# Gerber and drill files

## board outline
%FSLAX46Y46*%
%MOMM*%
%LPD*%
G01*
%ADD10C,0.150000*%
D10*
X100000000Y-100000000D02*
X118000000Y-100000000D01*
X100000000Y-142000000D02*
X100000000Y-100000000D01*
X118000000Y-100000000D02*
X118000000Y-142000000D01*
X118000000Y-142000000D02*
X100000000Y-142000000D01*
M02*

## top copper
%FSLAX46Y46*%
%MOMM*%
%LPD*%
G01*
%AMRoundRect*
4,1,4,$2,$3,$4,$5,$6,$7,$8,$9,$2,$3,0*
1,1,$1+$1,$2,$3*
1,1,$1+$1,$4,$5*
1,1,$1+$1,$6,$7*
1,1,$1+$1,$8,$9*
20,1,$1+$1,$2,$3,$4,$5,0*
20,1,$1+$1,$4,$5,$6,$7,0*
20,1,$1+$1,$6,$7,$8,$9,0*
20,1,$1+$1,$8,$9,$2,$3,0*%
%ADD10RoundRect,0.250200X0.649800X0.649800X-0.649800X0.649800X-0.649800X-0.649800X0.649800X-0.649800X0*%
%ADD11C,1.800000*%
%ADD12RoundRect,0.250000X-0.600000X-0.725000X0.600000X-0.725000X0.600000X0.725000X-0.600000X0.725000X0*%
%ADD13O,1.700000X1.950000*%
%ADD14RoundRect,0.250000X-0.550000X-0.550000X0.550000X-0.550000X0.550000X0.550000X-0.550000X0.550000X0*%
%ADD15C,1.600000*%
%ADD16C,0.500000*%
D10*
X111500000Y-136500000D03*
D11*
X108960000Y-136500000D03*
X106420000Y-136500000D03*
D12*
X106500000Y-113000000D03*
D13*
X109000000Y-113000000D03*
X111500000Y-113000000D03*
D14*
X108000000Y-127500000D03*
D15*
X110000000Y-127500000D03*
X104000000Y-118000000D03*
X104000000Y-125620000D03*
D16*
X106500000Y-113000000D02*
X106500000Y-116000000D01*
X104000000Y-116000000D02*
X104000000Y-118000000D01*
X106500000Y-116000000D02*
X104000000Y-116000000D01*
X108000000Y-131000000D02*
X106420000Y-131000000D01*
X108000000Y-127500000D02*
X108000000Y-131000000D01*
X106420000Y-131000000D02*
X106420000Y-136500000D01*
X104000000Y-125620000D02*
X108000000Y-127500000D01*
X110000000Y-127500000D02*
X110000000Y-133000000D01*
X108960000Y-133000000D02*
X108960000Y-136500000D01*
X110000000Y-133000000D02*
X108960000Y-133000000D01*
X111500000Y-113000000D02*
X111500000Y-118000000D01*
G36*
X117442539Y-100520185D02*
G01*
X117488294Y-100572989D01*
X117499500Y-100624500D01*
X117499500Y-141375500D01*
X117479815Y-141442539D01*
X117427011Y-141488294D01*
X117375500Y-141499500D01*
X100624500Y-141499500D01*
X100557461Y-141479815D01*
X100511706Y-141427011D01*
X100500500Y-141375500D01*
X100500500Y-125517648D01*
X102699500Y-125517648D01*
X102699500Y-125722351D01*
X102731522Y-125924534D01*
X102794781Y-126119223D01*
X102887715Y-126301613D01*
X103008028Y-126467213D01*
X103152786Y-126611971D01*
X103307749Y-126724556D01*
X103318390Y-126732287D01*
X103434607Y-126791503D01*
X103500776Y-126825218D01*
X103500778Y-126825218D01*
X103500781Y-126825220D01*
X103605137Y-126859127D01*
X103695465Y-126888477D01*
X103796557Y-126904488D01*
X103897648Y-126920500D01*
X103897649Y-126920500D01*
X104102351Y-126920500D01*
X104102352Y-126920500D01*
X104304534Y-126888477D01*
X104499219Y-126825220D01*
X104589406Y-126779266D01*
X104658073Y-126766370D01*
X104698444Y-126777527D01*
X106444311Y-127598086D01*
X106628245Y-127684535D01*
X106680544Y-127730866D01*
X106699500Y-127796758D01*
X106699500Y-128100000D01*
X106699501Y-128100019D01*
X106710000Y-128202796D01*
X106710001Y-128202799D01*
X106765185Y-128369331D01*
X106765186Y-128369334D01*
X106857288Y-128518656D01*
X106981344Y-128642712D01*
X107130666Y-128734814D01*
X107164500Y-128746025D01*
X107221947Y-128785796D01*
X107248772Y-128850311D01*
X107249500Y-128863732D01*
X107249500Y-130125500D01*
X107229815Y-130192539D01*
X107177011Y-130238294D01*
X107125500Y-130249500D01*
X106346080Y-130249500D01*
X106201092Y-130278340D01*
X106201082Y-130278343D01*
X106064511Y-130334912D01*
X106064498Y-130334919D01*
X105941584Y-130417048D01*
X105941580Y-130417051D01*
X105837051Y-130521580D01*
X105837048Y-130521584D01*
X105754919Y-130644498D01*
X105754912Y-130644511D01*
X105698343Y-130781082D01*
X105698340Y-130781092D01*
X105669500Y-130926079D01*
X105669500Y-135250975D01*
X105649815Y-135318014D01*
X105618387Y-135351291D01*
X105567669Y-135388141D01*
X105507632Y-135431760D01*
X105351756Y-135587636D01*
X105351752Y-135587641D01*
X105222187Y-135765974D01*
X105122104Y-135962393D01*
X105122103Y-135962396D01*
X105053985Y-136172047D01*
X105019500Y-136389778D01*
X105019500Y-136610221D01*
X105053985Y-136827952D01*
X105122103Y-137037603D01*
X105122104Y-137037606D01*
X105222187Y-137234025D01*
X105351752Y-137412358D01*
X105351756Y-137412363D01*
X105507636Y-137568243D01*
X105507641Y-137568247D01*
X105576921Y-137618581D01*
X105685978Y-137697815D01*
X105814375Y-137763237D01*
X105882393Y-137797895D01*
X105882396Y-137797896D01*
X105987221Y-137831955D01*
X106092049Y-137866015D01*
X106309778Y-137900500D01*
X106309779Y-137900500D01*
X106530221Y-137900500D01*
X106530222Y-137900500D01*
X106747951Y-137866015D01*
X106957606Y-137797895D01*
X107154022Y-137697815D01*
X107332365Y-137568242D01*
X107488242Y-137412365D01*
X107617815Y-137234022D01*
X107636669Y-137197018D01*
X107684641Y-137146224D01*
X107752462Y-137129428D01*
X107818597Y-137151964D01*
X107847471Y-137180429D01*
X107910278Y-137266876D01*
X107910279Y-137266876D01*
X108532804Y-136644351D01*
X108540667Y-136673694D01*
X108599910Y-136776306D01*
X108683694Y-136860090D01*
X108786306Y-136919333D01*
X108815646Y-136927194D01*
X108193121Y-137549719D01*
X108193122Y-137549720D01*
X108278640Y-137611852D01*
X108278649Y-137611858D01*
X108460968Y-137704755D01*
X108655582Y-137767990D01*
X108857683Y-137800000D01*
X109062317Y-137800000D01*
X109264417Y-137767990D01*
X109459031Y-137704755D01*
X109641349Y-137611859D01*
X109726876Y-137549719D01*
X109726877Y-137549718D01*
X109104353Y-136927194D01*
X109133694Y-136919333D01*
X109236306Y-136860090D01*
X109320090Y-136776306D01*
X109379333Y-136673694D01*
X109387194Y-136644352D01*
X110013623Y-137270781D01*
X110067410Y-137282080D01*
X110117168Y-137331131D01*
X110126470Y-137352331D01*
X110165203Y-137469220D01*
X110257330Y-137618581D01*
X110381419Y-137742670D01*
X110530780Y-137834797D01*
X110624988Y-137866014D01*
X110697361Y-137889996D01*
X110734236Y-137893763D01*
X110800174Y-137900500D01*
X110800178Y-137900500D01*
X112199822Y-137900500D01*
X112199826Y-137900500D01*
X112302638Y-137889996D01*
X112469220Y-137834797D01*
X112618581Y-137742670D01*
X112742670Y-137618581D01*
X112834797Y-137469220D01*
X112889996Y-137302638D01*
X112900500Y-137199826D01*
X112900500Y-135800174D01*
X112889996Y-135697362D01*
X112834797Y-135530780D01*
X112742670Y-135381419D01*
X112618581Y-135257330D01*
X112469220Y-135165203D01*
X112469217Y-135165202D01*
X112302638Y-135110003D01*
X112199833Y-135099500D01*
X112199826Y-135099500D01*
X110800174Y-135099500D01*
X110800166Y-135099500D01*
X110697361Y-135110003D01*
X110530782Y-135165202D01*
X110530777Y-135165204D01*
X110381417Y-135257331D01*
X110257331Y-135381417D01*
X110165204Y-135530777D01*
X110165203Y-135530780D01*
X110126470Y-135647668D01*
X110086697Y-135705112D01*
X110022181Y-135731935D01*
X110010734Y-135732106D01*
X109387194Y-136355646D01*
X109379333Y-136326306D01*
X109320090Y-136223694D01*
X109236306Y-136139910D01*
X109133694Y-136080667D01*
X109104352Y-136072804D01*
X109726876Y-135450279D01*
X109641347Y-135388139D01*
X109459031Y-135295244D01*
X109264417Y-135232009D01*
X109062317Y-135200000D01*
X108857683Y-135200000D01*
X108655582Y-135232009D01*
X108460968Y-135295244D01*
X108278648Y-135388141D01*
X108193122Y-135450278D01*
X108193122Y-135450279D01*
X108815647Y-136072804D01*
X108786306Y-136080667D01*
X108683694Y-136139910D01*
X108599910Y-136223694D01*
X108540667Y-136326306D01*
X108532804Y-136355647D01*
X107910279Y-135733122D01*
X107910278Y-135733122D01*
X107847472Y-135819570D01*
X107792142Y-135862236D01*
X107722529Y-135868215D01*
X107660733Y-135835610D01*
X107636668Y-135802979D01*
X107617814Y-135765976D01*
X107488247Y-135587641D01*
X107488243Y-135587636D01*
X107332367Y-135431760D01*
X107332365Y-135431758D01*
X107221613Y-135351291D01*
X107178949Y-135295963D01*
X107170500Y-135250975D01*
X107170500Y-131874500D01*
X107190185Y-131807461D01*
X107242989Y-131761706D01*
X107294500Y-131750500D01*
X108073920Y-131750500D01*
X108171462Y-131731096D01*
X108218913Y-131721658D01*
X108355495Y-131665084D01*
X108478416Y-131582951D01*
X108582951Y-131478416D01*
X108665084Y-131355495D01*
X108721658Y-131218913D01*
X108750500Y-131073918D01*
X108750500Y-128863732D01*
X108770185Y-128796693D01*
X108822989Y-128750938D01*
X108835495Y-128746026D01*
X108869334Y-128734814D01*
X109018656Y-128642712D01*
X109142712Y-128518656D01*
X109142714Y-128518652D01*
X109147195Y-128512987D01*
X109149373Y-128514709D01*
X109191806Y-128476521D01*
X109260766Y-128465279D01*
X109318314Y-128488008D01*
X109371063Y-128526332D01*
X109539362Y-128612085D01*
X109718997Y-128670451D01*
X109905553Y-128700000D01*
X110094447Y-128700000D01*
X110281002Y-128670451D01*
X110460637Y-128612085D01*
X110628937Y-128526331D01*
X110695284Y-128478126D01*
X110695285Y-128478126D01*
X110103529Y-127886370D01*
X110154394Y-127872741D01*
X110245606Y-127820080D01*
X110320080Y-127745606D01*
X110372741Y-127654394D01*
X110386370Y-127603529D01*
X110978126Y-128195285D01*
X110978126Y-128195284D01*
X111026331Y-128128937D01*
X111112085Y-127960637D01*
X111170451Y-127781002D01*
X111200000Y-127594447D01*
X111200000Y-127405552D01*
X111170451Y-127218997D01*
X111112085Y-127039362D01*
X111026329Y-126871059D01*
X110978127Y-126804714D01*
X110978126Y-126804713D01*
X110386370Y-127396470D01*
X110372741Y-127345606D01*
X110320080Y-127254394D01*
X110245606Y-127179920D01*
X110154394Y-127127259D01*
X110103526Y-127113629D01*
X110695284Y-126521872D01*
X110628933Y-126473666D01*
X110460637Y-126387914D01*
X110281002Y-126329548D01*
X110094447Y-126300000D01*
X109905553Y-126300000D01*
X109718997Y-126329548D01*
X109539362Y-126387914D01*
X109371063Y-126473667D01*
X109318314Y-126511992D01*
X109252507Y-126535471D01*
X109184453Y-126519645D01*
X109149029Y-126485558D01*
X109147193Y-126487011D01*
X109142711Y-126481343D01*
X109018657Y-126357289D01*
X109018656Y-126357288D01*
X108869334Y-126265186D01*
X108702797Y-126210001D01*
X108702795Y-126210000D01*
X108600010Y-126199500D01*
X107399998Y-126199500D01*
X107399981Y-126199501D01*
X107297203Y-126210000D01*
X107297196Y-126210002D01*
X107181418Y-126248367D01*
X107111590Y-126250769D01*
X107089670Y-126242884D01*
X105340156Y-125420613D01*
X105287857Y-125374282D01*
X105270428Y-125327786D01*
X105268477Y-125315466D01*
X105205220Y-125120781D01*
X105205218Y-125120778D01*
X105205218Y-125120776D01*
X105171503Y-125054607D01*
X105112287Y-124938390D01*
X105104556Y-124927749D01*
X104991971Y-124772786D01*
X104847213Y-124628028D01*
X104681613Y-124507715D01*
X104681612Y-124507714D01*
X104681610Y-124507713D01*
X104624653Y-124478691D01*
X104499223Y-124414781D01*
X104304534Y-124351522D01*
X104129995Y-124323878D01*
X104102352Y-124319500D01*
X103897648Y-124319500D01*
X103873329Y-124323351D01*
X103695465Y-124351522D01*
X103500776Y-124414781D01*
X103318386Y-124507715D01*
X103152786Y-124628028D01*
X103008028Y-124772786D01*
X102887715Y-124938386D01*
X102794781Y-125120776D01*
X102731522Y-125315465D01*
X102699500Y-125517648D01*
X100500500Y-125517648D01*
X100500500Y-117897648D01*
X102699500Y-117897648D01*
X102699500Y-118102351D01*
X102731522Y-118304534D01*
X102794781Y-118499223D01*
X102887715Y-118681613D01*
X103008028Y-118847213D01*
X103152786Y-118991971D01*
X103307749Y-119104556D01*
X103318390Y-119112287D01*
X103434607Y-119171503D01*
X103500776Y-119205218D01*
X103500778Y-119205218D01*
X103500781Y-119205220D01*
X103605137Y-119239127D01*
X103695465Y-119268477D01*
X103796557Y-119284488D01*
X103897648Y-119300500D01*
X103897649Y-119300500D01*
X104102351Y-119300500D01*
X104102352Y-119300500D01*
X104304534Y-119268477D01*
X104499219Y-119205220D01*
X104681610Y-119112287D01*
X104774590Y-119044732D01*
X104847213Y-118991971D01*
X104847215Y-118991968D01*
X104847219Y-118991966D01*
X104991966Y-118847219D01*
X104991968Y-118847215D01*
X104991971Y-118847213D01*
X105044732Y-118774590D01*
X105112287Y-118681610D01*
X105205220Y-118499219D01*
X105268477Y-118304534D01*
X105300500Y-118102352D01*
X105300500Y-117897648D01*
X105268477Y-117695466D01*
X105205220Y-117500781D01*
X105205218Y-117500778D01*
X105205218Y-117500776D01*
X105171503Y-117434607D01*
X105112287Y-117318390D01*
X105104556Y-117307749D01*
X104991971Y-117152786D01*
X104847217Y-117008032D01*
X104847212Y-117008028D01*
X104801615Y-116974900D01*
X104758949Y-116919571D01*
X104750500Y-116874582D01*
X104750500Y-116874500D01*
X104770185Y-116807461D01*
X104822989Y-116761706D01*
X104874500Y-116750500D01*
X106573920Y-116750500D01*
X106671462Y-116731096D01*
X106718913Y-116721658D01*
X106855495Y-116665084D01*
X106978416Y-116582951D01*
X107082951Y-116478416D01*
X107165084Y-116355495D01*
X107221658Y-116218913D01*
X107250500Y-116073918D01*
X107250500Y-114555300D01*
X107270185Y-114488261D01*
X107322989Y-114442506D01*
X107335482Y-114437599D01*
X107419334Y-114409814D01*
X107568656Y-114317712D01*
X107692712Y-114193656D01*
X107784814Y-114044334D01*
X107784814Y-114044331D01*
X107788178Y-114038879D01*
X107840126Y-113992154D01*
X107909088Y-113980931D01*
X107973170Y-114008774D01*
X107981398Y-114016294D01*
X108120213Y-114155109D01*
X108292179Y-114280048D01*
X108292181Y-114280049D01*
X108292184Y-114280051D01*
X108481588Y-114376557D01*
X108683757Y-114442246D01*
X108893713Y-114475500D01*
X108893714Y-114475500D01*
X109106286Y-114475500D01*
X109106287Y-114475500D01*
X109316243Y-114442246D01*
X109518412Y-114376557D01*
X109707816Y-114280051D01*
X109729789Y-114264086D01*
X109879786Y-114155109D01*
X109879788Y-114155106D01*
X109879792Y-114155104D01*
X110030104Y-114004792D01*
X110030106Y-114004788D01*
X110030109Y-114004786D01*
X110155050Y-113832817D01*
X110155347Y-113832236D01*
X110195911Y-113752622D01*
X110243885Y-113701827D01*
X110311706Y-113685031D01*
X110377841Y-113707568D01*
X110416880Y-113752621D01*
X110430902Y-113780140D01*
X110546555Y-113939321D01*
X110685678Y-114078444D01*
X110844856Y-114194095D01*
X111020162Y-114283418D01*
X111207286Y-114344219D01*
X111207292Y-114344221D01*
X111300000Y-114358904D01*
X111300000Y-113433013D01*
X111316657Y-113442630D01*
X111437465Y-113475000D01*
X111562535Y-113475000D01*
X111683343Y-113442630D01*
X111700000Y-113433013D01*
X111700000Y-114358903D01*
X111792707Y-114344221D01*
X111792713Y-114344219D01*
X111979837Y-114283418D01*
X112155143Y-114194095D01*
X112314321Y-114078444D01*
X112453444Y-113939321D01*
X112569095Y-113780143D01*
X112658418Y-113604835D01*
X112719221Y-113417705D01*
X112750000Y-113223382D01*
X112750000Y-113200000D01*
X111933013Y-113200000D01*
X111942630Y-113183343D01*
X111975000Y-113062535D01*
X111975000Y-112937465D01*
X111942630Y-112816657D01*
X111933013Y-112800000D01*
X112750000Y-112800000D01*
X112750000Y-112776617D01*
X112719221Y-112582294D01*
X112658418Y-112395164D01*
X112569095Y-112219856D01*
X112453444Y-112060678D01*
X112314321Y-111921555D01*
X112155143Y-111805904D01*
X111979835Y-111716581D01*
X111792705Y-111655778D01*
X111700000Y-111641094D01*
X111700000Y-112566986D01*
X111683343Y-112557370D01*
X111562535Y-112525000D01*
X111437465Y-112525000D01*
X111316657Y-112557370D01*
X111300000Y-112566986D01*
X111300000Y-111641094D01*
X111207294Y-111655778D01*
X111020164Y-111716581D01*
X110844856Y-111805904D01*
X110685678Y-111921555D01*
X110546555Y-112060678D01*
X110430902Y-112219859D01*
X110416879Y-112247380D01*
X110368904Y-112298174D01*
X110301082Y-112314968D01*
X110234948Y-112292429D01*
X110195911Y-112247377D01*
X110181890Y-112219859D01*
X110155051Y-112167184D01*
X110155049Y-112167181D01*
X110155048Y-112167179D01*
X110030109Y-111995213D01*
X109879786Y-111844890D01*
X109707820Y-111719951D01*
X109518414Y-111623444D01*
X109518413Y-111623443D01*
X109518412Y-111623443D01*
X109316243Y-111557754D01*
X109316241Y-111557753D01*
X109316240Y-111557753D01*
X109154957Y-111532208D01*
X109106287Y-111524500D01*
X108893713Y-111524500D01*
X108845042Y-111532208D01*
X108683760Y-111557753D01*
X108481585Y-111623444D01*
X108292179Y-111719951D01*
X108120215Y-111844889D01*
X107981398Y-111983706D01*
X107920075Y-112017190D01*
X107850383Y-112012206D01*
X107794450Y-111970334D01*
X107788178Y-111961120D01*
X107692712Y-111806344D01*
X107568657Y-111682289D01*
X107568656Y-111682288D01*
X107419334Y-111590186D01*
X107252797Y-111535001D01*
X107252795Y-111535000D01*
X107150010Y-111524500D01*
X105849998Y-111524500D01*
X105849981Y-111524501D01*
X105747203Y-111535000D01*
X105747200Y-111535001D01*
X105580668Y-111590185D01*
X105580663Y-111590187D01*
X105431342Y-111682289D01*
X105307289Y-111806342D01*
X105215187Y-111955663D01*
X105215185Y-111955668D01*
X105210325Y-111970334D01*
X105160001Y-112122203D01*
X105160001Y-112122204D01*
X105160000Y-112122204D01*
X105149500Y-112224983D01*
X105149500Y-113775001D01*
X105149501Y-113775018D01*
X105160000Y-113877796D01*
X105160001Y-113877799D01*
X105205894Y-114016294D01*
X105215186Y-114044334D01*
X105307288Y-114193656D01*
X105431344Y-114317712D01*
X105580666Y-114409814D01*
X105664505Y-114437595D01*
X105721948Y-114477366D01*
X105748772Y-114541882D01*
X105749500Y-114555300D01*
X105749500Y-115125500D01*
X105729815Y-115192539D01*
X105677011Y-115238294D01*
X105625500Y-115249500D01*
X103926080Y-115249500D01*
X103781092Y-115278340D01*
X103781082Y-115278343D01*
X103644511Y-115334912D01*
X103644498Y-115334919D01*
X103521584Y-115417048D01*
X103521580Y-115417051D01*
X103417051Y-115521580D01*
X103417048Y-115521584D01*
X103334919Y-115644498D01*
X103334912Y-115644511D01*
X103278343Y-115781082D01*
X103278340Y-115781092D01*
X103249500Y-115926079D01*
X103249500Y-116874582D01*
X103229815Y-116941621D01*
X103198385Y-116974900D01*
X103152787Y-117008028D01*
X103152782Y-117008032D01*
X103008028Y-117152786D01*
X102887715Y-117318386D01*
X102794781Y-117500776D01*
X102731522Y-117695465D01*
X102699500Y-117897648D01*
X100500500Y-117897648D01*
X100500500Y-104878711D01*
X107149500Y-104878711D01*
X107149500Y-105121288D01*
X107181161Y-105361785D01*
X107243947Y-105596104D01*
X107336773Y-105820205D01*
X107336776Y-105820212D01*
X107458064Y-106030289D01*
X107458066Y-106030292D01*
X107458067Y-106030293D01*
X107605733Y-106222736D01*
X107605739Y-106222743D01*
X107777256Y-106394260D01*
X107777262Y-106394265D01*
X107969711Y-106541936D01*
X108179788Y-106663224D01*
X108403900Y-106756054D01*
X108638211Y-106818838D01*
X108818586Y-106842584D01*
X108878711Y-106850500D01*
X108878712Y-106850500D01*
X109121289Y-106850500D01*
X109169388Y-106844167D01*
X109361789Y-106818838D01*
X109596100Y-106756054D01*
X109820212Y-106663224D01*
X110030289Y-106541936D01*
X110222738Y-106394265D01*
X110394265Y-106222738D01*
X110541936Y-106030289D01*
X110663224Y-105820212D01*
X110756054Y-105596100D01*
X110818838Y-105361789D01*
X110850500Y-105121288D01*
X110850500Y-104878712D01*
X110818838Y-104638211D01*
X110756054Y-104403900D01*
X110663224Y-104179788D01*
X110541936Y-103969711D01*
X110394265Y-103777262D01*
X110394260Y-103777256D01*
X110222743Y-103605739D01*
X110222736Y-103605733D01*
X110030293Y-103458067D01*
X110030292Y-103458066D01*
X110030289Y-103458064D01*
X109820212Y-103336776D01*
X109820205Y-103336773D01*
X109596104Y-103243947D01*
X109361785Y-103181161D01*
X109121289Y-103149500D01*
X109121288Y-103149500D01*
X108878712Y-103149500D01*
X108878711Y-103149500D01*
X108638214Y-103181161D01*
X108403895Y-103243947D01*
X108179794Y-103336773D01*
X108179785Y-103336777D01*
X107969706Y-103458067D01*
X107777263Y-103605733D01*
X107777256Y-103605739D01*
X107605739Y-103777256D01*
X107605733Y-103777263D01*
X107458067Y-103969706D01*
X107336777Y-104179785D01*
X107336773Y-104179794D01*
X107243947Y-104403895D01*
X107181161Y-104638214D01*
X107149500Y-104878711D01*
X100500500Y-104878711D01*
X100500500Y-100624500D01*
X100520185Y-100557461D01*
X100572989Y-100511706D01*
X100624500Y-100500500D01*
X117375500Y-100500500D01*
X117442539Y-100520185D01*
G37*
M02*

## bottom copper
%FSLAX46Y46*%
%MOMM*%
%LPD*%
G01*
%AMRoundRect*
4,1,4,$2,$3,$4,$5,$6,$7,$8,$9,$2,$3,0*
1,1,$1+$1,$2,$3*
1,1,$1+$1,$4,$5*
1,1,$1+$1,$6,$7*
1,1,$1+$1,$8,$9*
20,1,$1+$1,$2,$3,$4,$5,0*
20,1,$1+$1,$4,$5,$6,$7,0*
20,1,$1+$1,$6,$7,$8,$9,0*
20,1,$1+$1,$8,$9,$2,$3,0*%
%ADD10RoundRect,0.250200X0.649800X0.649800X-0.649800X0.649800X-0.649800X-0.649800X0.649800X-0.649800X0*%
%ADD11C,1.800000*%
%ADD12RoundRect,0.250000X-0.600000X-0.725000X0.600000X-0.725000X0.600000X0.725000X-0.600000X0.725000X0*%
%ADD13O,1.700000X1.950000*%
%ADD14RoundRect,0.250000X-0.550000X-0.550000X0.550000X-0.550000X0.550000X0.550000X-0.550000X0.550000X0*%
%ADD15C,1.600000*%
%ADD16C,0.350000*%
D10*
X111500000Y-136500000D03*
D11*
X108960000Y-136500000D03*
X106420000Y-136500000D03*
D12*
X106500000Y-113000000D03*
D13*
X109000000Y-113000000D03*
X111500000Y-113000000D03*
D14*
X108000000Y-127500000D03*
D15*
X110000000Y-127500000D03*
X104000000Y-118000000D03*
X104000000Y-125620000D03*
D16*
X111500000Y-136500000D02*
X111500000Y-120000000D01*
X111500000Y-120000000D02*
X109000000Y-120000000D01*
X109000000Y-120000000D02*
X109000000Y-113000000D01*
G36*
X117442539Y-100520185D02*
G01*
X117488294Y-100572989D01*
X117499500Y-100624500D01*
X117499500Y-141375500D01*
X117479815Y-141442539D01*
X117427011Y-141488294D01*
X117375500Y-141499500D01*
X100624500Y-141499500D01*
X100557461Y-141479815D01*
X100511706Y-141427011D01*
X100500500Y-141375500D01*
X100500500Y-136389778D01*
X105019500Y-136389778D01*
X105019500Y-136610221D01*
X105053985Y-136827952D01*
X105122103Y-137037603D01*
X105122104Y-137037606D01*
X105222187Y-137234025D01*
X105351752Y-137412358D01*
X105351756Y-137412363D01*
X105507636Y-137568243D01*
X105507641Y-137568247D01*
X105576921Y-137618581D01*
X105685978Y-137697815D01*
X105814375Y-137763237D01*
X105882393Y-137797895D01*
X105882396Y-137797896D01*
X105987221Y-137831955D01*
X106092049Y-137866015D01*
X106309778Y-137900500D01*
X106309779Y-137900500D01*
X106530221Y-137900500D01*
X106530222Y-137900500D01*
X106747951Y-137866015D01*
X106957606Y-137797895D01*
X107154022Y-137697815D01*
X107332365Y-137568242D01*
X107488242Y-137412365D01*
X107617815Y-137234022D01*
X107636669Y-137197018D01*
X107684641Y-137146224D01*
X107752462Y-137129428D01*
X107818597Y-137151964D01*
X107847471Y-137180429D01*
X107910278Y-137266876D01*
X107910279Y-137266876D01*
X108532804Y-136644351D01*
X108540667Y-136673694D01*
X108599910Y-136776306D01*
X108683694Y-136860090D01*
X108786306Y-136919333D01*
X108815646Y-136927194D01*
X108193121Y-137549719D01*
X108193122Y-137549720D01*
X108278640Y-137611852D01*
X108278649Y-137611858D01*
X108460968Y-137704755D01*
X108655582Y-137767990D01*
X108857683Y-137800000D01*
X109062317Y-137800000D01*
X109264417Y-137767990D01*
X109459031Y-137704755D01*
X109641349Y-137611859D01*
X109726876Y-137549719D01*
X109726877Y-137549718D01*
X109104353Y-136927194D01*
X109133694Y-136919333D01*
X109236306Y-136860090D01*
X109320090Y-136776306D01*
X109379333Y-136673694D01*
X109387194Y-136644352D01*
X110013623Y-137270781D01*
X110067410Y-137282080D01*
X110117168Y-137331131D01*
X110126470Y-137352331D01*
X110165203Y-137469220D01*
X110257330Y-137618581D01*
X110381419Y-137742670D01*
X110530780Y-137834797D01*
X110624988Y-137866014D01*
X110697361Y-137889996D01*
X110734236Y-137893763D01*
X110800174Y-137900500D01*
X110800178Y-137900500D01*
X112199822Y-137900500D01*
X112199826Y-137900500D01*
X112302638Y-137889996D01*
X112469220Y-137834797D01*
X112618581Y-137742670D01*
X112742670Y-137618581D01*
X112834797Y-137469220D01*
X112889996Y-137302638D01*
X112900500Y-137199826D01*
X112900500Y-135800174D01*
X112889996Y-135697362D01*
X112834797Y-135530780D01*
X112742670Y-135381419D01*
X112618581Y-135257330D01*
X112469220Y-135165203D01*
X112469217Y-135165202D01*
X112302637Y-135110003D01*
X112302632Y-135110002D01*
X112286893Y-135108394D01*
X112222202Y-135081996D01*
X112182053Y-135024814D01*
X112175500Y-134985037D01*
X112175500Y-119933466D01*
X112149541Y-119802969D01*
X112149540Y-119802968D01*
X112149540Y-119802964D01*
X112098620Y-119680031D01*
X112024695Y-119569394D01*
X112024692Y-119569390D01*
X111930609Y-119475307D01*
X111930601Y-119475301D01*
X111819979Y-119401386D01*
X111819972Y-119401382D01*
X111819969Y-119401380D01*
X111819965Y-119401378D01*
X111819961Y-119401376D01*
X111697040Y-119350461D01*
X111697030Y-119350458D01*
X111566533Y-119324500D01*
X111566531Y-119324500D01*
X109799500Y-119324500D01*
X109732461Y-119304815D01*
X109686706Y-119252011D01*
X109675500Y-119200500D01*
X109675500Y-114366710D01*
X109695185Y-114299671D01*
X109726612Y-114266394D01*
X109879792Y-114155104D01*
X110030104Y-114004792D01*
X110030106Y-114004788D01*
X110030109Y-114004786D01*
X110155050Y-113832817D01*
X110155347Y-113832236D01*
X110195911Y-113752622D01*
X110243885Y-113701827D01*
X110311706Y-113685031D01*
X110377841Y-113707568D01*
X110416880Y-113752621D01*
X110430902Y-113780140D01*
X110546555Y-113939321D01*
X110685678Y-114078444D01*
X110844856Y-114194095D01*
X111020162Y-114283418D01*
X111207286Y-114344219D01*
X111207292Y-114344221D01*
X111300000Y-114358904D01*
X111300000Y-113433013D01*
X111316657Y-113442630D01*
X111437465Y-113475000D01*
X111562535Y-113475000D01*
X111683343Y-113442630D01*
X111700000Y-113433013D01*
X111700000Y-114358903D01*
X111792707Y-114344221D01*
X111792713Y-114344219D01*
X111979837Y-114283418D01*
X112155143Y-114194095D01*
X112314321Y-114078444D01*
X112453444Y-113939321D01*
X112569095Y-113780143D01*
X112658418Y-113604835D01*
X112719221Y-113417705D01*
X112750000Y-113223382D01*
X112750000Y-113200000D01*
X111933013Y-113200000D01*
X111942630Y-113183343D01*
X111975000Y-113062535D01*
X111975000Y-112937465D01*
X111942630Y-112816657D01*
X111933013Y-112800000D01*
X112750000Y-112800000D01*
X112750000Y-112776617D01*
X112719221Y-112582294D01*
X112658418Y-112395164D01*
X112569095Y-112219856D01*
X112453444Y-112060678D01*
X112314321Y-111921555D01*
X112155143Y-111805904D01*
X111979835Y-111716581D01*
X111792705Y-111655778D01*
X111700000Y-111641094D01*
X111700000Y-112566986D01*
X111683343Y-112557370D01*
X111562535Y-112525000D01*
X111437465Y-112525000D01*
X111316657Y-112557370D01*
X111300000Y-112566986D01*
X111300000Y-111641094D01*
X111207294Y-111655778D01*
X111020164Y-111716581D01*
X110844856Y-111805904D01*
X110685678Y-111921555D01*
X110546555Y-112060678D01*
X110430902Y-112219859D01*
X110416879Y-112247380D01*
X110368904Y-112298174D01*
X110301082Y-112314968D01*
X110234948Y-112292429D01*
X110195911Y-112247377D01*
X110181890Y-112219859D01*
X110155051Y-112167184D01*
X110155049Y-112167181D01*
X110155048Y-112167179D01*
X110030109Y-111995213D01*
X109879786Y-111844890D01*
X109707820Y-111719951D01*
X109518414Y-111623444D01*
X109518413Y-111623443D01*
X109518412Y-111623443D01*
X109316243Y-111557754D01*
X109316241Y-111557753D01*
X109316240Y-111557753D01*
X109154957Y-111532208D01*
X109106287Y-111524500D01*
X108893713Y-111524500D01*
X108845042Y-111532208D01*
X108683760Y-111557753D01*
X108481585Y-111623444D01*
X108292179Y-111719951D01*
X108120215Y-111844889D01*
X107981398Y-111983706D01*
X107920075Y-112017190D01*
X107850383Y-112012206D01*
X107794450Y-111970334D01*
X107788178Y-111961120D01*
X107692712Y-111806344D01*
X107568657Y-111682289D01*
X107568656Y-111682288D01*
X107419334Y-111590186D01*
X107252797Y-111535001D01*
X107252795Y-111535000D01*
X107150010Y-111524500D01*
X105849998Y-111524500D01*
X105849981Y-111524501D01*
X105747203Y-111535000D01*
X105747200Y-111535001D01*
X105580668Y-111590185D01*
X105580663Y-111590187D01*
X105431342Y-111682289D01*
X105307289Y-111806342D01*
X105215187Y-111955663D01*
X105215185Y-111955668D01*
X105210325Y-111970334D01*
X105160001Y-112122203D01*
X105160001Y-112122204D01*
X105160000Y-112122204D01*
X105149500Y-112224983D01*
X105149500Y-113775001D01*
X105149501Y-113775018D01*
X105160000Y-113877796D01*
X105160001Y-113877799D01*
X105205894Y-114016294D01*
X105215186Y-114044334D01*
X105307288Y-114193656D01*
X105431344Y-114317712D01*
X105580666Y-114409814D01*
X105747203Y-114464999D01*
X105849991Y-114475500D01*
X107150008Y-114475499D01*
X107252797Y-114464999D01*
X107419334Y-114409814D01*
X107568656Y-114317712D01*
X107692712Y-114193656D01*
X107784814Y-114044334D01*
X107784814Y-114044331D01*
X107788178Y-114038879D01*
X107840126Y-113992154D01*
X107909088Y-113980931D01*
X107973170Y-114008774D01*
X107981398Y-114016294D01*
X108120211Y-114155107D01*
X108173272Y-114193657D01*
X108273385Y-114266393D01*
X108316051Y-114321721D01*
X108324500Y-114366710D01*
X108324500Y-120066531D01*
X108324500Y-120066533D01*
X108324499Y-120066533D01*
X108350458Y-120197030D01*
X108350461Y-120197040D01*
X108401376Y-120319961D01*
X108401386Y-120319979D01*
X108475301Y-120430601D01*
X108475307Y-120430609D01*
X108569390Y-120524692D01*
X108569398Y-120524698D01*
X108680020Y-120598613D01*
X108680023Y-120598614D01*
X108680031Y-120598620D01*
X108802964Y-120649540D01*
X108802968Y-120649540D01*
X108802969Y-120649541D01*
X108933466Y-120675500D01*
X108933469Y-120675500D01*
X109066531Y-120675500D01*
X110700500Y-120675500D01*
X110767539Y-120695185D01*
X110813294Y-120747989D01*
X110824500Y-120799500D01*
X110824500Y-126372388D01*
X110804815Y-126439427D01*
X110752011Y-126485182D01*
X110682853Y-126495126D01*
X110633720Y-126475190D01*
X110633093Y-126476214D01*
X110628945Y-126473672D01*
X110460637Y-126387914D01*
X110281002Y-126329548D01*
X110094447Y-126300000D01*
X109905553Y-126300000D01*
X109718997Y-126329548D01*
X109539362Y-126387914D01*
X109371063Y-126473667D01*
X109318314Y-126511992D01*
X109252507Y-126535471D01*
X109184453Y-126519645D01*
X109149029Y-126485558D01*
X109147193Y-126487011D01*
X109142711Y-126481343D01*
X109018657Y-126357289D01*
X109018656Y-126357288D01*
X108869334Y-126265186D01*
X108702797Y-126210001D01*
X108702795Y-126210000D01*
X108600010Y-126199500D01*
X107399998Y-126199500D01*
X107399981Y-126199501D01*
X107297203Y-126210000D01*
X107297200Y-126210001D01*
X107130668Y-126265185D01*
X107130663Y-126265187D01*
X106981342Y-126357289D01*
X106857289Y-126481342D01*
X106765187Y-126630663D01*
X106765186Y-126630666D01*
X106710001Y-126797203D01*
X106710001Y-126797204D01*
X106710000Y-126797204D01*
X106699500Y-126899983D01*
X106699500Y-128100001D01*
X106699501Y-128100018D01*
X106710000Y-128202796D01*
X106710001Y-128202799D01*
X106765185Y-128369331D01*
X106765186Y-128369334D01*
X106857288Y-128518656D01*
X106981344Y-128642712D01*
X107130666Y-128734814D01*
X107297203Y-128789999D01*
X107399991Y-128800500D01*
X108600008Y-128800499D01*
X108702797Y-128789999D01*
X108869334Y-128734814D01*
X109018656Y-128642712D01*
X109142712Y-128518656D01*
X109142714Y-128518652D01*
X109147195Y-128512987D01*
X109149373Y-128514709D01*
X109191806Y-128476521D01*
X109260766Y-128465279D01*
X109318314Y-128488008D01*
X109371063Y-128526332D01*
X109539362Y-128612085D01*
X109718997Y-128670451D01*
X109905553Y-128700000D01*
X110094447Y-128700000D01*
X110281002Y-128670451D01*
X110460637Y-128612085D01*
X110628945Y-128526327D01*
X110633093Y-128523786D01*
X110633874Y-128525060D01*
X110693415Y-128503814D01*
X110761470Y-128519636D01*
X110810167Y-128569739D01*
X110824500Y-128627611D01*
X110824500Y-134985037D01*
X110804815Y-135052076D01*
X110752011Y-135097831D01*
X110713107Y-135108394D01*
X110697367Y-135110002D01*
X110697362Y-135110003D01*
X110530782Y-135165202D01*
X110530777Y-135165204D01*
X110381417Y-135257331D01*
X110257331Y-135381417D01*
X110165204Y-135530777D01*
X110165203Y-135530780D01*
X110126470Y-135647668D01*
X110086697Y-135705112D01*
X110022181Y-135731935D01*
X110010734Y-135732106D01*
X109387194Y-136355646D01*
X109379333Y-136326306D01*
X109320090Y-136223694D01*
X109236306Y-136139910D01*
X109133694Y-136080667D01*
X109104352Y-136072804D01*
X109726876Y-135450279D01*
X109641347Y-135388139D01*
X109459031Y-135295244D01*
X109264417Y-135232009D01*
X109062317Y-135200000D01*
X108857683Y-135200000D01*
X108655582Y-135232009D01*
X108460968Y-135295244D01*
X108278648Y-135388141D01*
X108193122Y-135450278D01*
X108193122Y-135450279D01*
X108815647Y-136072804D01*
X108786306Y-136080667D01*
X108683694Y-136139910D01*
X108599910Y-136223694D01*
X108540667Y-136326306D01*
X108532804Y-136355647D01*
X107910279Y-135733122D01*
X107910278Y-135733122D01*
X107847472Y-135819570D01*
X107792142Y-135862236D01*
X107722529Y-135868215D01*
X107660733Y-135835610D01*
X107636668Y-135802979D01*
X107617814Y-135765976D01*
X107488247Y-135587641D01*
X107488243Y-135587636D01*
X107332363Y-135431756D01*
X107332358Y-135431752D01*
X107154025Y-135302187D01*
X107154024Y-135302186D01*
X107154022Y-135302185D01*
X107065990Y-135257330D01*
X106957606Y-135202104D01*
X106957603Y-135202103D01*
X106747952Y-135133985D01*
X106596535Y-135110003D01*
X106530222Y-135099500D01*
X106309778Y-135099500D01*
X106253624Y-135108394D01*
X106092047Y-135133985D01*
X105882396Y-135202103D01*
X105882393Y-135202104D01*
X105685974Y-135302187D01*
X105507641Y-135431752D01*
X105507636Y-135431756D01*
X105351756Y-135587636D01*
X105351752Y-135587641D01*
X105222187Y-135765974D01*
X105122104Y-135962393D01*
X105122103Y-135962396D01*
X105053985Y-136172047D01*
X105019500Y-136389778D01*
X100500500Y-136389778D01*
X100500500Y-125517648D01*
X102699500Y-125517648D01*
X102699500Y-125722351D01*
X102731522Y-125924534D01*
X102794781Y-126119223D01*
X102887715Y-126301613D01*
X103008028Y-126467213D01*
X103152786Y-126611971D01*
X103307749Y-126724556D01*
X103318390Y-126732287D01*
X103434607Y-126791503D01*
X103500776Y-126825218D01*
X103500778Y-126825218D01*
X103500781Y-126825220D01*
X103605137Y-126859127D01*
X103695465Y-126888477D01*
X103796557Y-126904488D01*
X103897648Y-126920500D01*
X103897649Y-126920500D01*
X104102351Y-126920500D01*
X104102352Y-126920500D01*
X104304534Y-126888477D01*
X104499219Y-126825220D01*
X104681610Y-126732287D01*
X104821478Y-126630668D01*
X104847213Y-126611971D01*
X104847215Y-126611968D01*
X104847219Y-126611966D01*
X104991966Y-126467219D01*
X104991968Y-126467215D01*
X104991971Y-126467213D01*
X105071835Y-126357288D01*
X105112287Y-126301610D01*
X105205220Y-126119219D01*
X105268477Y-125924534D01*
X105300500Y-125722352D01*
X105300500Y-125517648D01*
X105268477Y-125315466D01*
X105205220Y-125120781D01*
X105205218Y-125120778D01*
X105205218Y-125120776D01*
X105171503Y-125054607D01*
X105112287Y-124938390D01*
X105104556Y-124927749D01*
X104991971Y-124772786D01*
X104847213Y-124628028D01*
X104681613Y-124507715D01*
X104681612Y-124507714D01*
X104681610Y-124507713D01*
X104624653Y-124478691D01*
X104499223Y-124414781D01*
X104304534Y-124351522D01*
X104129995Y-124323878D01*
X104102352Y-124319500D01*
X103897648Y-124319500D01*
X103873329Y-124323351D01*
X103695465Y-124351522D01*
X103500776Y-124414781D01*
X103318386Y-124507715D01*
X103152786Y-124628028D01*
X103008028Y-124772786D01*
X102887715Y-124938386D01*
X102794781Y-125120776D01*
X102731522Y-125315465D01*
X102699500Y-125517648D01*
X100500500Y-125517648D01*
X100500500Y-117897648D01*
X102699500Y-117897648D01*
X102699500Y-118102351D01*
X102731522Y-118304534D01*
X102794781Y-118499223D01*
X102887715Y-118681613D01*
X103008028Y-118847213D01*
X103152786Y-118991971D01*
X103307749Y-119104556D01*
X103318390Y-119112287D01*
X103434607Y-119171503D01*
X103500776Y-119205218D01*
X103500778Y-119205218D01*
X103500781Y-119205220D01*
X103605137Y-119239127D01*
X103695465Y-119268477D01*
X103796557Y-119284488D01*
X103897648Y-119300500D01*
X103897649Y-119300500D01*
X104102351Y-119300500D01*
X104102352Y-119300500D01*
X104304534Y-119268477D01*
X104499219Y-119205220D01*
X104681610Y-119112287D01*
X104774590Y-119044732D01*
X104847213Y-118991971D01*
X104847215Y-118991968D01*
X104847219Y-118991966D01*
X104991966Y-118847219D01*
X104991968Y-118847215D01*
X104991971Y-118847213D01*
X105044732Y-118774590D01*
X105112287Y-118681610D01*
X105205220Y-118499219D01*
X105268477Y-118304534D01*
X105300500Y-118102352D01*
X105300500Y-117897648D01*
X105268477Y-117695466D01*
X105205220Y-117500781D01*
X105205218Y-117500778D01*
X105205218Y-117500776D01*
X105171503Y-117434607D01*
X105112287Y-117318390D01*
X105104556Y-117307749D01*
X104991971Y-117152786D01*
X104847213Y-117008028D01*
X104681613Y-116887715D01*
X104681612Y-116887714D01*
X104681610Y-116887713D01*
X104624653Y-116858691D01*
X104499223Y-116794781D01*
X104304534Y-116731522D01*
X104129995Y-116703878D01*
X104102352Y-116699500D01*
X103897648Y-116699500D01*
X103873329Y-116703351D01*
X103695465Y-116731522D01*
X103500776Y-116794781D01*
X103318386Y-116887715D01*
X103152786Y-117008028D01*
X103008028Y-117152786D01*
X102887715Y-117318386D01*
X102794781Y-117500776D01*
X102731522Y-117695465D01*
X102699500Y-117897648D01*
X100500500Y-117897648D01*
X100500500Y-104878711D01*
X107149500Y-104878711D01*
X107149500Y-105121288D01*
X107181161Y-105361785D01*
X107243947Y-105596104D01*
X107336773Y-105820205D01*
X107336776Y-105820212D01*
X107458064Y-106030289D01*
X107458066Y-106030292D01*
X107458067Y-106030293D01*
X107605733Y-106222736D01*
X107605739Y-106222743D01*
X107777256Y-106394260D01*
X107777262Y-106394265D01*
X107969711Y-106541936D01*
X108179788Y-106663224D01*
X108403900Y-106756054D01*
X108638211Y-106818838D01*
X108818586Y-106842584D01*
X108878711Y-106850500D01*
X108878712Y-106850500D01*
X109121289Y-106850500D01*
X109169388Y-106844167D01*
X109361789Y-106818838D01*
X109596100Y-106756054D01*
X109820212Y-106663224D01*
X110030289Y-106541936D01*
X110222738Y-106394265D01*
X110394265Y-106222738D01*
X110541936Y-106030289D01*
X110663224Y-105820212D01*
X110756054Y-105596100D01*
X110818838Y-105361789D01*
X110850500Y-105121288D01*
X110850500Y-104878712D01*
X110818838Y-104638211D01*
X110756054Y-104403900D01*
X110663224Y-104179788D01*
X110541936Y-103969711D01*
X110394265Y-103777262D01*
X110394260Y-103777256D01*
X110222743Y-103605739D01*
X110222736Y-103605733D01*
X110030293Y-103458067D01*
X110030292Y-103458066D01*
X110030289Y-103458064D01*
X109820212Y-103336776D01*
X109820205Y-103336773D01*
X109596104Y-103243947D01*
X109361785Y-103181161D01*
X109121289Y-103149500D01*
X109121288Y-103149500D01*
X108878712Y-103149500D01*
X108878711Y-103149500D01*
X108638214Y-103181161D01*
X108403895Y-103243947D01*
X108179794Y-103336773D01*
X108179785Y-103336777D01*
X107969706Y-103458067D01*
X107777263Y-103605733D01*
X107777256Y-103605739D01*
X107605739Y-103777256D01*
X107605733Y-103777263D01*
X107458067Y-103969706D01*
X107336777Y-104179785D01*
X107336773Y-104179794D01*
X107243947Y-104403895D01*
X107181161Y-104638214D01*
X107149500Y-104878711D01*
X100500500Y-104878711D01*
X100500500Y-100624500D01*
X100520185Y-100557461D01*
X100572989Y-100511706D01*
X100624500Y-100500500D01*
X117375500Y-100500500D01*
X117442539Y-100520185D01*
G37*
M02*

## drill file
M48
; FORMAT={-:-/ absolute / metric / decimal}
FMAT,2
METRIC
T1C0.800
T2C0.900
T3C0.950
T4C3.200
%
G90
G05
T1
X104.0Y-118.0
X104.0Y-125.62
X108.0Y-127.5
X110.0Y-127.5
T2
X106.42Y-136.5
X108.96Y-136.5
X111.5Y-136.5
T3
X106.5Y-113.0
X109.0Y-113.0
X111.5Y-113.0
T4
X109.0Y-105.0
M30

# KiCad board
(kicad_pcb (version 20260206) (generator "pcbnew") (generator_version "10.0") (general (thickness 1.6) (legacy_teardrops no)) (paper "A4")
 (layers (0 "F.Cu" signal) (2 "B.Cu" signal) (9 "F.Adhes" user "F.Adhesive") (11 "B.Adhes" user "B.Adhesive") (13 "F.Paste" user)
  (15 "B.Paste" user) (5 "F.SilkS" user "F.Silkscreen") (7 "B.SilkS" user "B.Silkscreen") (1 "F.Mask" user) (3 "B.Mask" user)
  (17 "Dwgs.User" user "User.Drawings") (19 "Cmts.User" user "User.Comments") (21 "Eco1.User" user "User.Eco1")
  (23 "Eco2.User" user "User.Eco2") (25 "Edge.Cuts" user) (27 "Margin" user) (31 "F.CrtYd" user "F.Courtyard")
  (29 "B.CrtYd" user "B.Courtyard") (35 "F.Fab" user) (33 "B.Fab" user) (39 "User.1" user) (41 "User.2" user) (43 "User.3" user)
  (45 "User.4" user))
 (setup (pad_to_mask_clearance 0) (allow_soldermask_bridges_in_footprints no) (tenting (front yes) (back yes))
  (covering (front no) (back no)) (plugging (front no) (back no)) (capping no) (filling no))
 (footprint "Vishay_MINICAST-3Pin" (layer "F.Cu") (at 111.5 136.5 180)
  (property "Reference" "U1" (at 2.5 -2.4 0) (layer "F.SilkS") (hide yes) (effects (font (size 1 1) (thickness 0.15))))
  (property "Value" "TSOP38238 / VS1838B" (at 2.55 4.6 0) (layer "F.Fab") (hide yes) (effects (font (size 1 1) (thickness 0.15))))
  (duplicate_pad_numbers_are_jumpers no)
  (pad "1" thru_hole roundrect (at 0 0 180) (size 1.8 1.8) (drill 0.9) (layers "*.Cu" "*.Mask") (remove_unused_layers no)
   (roundrect_rratio 0.139) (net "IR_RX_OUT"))
  (pad "2" thru_hole circle (at 2.54 0 180) (size 1.8 1.8) (drill 0.9) (layers "*.Cu" "*.Mask") (remove_unused_layers no) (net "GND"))
  (pad "3" thru_hole circle (at 5.08 0 180) (size 1.8 1.8) (drill 0.9) (layers "*.Cu" "*.Mask") (remove_unused_layers no) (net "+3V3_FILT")))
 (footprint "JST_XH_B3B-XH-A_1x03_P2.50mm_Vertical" (layer "F.Cu") (at 106.5 113)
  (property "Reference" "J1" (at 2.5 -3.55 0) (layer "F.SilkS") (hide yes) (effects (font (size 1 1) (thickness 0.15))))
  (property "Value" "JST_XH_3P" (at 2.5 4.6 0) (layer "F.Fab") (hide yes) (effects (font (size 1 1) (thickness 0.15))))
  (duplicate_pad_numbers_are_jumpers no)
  (pad "1" thru_hole roundrect (at 0 0) (size 1.7 1.95) (drill 0.95) (layers "*.Cu" "*.Mask") (remove_unused_layers no)
   (roundrect_rratio 0.147059) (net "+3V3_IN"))
  (pad "2" thru_hole oval (at 2.5 0) (size 1.7 1.95) (drill 0.95) (layers "*.Cu" "*.Mask") (remove_unused_layers no) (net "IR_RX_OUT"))
  (pad "3" thru_hole oval (at 5 0) (size 1.7 1.95) (drill 0.95) (layers "*.Cu" "*.Mask") (remove_unused_layers no) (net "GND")))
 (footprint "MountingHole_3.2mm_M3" (layer "F.Cu") (at 109 105)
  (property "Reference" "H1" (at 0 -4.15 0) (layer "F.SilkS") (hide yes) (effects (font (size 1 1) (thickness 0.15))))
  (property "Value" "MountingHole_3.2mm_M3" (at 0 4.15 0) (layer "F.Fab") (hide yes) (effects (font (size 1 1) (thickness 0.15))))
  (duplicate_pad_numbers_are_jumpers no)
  (pad "" np_thru_hole circle (at 0 0) (size 3.2 3.2) (drill 3.2) (layers "*.Cu" "*.Mask")))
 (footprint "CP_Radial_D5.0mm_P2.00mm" (layer "F.Cu") (at 108 127.5)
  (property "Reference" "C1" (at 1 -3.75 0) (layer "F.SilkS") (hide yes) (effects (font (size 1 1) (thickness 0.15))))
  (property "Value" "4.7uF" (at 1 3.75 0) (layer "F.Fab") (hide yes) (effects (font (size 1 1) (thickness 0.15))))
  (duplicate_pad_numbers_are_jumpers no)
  (pad "1" thru_hole roundrect (at 0 0) (size 1.6 1.6) (drill 0.8) (layers "*.Cu" "*.Mask") (remove_unused_layers no)
   (roundrect_rratio 0.15625) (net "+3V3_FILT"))
  (pad "2" thru_hole circle (at 2 0) (size 1.6 1.6) (drill 0.8) (layers "*.Cu" "*.Mask") (remove_unused_layers no) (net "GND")))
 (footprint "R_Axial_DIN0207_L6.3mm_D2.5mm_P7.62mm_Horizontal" (layer "F.Cu") (at 104 118 -90)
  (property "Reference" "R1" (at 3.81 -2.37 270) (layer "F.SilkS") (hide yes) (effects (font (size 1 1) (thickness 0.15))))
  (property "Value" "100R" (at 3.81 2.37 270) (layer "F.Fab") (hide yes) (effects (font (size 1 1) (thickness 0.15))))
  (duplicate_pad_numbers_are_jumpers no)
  (pad "1" thru_hole circle (at 0 0 270) (size 1.6 1.6) (drill 0.8) (layers "*.Cu" "*.Mask") (remove_unused_layers no) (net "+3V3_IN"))
  (pad "2" thru_hole circle (at 7.62 0 270) (size 1.6 1.6) (drill 0.8) (layers "*.Cu" "*.Mask") (remove_unused_layers no) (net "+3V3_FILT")))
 (gr_line (start 100 100) (end 118 100) (stroke (width 0.15) (type default)) (layer "Edge.Cuts"))
 (gr_line (start 100 142) (end 100 100) (stroke (width 0.15) (type default)) (layer "Edge.Cuts"))
 (gr_line (start 118 100) (end 118 142) (stroke (width 0.15) (type default)) (layer "Edge.Cuts"))
 (gr_line (start 118 142) (end 100 142) (stroke (width 0.15) (type default)) (layer "Edge.Cuts"))
 (segment (start 106.5 113) (end 106.5 116) (width 0.5) (layer "F.Cu") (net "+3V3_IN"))
 (segment (start 104 116) (end 104 118) (width 0.5) (layer "F.Cu") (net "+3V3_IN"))
 (segment (start 106.5 116) (end 104 116) (width 0.5) (layer "F.Cu") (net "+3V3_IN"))
 (segment (start 108 131) (end 106.42 131) (width 0.5) (layer "F.Cu") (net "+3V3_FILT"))
 (segment (start 108 127.5) (end 108 131) (width 0.5) (layer "F.Cu") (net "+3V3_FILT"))
 (segment (start 106.42 131) (end 106.42 136.5) (width 0.5) (layer "F.Cu") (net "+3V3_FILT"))
 (segment (start 104 125.62) (end 108 127.5) (width 0.5) (layer "F.Cu") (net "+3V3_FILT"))
 (segment (start 111.5 136.5) (end 111.5 120) (width 0.35) (layer "B.Cu") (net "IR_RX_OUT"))
 (segment (start 111.5 120) (end 109 120) (width 0.35) (layer "B.Cu") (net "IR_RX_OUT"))
 (segment (start 109 120) (end 109 113) (width 0.35) (layer "B.Cu") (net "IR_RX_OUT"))
 (segment (start 110 127.5) (end 110 133) (width 0.5) (layer "F.Cu") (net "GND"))
 (segment (start 108.96 133) (end 108.96 136.5) (width 0.5) (layer "F.Cu") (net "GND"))
 (segment (start 110 133) (end 108.96 133) (width 0.5) (layer "F.Cu") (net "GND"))
 (segment (start 111.5 113) (end 111.5 118) (width 0.5) (layer "F.Cu") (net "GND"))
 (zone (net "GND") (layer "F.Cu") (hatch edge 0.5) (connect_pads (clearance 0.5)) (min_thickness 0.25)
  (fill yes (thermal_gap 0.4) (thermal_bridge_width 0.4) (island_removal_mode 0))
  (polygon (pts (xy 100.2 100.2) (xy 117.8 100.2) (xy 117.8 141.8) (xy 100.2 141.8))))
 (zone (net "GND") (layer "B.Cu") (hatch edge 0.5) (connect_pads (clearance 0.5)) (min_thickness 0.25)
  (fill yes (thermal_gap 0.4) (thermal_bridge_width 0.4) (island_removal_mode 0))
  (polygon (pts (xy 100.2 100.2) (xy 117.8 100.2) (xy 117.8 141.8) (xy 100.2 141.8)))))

